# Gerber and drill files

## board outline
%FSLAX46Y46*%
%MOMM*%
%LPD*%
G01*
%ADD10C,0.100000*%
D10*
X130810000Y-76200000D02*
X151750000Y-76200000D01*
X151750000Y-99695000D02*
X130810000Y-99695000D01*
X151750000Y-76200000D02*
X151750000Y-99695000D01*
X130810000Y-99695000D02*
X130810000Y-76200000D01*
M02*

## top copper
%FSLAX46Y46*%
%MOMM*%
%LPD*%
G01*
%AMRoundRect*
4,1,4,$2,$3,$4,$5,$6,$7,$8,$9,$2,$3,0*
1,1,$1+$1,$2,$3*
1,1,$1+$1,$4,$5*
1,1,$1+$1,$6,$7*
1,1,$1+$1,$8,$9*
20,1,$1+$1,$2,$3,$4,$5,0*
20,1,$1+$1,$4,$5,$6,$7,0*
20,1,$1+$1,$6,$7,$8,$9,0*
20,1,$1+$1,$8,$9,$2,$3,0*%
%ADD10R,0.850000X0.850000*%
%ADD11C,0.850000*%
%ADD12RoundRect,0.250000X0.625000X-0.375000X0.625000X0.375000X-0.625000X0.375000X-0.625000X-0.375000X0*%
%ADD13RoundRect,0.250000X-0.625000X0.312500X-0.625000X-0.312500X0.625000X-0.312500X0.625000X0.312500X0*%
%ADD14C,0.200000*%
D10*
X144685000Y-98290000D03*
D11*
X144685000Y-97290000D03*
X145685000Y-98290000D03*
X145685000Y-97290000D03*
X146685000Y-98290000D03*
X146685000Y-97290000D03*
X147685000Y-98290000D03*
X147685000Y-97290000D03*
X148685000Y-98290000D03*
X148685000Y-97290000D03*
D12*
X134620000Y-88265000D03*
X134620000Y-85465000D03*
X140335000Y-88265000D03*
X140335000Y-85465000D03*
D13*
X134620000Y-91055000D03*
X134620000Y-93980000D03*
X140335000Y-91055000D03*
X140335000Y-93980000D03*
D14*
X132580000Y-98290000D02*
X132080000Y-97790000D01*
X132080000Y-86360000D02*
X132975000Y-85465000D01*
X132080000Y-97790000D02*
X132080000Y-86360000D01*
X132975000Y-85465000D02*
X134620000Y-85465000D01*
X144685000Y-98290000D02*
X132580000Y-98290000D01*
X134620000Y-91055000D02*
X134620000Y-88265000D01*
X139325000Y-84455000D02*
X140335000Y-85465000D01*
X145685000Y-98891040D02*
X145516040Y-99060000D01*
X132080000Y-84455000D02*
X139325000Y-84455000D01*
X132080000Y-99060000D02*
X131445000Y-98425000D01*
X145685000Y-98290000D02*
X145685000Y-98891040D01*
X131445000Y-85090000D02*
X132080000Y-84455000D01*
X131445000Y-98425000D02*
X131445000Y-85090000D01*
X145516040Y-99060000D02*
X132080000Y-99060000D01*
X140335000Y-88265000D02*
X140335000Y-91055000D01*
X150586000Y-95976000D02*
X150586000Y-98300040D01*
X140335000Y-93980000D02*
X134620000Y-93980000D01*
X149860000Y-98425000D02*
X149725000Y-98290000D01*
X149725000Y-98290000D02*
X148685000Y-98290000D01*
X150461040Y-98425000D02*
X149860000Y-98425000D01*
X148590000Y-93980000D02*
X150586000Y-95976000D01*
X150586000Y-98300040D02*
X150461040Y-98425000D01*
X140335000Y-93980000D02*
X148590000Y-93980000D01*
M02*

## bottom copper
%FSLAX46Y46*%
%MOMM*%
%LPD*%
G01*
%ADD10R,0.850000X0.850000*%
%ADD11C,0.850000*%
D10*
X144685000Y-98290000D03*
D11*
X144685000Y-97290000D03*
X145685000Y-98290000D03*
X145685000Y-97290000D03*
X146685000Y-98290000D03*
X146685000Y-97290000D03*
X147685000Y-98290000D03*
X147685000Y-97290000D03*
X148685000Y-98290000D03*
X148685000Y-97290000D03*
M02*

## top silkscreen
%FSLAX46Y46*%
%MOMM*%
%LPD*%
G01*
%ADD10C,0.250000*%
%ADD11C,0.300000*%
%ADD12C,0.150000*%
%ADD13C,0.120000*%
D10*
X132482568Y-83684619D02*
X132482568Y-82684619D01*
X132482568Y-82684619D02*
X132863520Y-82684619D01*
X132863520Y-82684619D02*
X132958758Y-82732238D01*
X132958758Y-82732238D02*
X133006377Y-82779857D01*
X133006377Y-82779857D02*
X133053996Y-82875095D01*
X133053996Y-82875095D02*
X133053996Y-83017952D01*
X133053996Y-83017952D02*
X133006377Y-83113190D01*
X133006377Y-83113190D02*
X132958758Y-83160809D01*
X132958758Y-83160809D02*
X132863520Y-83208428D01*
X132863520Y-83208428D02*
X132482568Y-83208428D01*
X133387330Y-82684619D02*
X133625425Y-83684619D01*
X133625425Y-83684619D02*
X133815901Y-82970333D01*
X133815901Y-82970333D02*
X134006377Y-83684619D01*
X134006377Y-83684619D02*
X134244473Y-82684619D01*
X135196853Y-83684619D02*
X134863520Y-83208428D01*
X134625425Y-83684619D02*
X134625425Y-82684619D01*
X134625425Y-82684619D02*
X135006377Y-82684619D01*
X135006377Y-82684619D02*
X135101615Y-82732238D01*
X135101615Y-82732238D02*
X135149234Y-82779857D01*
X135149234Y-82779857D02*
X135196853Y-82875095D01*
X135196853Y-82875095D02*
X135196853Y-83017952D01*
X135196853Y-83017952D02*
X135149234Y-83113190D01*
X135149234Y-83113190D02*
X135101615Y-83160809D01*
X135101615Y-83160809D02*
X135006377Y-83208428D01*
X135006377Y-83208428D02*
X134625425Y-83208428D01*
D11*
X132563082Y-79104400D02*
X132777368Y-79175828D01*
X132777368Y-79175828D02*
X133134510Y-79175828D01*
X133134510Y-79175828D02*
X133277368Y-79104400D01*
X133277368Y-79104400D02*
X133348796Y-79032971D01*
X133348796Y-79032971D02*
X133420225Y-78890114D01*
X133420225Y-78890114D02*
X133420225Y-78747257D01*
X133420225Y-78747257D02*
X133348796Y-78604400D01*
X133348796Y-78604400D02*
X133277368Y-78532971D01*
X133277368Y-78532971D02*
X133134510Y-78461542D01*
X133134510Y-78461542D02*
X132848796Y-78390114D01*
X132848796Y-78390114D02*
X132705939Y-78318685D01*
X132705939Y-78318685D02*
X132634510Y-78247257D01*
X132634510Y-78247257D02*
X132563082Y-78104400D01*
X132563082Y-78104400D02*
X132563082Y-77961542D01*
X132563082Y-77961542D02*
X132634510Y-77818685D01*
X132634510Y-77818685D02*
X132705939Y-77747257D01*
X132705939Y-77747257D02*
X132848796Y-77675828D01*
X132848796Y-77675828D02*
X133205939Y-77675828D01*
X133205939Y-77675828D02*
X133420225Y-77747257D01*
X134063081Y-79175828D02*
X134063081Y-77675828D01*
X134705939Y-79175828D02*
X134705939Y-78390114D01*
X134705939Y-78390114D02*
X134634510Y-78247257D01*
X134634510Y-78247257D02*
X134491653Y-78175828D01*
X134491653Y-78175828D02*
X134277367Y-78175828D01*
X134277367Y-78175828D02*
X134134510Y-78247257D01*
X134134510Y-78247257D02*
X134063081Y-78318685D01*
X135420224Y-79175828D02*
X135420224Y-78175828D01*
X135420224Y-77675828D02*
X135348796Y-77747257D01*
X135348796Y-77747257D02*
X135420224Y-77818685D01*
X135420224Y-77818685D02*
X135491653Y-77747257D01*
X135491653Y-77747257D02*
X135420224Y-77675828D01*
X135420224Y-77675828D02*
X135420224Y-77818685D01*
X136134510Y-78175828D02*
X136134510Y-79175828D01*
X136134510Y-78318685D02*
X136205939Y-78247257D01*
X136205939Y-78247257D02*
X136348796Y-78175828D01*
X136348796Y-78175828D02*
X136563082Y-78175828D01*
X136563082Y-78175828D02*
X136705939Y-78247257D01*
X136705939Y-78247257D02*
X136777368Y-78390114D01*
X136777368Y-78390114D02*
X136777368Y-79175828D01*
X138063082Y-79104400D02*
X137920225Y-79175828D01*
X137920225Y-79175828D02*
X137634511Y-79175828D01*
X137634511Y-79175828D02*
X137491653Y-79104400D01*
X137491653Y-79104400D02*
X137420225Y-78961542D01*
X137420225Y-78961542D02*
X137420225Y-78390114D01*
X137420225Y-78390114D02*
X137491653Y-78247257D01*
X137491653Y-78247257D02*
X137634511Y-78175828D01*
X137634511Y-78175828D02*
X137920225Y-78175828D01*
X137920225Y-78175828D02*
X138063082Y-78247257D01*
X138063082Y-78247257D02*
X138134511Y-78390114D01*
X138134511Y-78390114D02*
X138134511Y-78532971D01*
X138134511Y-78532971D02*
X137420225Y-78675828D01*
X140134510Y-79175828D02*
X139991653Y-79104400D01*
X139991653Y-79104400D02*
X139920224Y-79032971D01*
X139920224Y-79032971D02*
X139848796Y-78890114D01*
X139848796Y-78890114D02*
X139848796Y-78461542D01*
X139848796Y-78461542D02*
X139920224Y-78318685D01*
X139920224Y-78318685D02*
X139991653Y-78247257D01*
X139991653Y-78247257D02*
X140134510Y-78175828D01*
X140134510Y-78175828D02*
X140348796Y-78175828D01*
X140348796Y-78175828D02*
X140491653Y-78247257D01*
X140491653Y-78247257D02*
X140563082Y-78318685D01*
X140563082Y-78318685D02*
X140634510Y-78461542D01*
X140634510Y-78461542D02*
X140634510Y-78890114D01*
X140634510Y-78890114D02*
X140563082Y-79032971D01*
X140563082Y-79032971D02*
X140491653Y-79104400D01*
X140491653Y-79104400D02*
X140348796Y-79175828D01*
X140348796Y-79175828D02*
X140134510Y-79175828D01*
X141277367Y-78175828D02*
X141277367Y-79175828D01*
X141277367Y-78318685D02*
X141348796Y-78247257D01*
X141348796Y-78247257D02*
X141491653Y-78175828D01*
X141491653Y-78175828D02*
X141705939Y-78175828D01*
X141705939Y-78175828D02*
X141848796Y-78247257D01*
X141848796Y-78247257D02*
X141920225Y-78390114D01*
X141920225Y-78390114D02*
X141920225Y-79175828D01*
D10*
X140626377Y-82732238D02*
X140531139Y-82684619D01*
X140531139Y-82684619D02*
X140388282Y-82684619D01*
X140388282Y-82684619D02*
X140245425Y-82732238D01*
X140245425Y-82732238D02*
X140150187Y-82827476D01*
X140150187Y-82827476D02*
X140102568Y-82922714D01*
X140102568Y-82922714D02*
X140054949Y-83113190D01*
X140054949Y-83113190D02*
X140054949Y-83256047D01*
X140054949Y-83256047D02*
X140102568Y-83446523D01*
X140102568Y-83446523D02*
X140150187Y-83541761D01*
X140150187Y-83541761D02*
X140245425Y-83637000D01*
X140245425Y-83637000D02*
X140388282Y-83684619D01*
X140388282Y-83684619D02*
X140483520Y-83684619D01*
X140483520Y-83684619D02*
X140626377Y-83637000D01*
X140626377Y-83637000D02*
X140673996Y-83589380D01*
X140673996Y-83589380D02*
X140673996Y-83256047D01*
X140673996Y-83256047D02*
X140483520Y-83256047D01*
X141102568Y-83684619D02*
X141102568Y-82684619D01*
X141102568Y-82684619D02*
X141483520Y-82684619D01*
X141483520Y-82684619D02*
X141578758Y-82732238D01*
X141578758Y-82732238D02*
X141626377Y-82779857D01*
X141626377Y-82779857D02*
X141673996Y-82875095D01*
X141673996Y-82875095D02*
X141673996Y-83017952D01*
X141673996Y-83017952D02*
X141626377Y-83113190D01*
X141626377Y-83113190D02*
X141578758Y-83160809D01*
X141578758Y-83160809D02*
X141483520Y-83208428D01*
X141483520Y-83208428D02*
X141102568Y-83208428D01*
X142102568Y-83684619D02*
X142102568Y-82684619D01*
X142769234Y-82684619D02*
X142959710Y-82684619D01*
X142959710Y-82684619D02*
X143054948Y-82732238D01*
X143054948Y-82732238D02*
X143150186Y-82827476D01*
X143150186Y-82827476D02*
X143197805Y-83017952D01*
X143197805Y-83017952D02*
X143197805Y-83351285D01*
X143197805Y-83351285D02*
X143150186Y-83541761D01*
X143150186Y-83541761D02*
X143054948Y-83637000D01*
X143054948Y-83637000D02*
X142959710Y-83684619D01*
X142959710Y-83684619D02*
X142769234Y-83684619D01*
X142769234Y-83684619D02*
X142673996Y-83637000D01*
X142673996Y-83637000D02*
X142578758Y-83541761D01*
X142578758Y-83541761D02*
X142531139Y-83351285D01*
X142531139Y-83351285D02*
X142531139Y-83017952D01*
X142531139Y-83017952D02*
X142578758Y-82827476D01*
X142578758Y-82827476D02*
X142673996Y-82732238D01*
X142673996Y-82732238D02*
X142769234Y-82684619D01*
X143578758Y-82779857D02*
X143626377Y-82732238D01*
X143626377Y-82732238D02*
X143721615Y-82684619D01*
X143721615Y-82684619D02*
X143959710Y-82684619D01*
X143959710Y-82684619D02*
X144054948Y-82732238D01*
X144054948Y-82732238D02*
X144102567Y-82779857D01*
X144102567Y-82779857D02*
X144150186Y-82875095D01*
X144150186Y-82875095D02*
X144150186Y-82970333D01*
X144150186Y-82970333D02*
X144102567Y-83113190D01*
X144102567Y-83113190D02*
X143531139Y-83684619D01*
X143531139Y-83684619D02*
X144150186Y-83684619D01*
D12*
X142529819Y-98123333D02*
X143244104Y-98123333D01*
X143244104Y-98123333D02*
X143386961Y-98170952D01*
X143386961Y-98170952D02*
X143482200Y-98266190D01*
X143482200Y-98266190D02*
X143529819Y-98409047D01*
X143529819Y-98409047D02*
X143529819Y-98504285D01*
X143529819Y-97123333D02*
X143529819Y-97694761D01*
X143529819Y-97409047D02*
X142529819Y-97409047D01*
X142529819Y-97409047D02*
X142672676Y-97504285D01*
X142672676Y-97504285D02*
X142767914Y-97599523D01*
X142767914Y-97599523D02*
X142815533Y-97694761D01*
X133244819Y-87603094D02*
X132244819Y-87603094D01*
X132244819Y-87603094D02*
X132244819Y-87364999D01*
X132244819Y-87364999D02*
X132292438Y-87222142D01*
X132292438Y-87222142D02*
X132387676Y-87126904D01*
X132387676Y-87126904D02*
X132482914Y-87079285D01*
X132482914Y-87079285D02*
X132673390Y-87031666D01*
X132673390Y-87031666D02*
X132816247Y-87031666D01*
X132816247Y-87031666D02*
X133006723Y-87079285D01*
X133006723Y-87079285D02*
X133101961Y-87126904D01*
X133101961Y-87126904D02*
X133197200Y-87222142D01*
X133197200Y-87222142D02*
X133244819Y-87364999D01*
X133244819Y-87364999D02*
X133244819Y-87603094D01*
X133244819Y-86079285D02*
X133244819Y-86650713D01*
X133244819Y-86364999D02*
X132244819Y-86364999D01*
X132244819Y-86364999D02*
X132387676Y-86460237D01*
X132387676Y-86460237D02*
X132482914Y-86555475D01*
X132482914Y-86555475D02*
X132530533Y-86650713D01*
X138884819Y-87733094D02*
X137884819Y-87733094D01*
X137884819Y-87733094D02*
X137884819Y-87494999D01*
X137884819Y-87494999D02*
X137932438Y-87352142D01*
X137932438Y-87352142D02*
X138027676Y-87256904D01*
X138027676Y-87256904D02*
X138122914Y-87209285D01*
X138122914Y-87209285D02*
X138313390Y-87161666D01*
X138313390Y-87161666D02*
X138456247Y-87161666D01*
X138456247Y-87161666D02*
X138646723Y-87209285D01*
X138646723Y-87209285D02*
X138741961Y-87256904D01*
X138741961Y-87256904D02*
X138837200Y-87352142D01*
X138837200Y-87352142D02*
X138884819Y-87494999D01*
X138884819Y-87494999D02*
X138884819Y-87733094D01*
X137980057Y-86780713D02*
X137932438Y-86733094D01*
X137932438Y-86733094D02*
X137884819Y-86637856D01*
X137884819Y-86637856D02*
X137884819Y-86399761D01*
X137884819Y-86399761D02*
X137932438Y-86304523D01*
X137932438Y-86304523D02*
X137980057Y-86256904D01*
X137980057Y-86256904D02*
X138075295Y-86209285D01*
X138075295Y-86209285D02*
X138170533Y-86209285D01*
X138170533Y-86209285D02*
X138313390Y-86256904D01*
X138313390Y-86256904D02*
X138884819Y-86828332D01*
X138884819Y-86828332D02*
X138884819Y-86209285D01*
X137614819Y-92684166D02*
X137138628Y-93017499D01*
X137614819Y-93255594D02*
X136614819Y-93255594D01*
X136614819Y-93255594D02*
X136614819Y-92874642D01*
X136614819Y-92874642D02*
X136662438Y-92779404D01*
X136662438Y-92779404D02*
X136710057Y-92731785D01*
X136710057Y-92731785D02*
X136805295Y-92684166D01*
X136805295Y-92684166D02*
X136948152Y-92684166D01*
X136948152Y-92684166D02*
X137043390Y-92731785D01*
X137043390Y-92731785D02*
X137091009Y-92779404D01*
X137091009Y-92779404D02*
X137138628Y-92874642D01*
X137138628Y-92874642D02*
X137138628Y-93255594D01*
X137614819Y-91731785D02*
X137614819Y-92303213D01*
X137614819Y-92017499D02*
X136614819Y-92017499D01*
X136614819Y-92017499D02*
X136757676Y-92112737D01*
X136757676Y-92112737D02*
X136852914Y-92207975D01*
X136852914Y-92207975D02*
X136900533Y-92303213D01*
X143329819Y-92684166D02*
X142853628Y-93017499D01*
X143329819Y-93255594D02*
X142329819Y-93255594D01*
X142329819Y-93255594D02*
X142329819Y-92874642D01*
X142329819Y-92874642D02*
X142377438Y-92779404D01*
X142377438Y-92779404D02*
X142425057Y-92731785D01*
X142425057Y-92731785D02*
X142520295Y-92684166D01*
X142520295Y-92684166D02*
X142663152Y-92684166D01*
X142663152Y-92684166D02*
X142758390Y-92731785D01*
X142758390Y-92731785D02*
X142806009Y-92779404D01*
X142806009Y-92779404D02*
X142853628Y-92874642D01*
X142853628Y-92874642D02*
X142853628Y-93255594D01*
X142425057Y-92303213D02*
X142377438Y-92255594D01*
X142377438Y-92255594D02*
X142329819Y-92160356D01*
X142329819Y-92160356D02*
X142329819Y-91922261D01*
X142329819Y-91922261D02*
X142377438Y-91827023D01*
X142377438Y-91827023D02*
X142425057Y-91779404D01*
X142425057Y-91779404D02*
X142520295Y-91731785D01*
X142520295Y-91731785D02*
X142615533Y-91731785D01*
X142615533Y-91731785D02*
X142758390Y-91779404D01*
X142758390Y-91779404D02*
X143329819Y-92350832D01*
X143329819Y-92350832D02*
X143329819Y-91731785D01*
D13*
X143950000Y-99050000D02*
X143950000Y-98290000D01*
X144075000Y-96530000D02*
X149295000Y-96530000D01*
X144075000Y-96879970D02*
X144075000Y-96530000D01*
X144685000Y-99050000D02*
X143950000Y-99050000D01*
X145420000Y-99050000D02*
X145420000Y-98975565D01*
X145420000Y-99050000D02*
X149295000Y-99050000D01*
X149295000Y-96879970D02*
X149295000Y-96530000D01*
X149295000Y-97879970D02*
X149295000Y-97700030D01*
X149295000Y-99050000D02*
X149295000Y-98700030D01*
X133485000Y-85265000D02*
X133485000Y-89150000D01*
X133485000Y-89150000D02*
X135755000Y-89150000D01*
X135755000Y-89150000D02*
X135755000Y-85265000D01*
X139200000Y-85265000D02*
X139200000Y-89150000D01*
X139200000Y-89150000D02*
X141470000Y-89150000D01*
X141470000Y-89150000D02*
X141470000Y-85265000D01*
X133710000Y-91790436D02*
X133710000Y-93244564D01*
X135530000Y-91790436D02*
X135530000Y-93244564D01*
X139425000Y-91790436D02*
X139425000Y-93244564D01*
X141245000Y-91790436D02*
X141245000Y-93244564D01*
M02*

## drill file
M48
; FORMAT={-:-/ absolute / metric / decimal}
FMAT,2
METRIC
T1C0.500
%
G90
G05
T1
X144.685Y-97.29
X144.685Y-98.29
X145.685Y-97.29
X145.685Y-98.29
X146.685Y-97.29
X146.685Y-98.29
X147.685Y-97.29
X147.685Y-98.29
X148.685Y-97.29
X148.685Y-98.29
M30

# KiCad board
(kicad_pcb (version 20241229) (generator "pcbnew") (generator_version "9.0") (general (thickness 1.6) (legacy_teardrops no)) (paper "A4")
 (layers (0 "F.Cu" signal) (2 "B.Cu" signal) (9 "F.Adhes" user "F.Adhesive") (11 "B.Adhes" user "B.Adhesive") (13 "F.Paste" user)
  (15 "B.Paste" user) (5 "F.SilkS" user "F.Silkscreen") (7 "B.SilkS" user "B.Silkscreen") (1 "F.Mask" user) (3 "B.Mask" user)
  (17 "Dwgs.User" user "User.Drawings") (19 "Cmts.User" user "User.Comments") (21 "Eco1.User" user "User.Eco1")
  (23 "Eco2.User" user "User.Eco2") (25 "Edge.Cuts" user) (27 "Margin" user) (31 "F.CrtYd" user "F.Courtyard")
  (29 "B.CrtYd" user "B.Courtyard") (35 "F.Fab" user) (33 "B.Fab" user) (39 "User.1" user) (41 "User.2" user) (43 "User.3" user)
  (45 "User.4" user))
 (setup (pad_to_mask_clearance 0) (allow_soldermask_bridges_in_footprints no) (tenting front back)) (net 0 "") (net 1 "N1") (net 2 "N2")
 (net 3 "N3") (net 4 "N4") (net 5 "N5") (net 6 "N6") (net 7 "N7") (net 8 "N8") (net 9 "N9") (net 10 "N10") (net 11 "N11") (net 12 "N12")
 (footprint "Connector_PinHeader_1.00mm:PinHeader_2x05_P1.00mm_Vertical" (layer "F.Cu") (at 144.685 98.29 90)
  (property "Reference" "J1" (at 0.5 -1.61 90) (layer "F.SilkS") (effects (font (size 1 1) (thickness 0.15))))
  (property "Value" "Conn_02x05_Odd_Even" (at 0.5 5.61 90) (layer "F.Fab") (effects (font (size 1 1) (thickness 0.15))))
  (fp_line (start -0.76 -0.735) (end 0 -0.735) (stroke (width 0.12) (type solid)) (layer "F.SilkS"))
  (fp_line (start 1.76 -0.61) (end 1.76 4.61) (stroke (width 0.12) (type solid)) (layer "F.SilkS"))
  (fp_line (start 1.41003 -0.61) (end 1.76 -0.61) (stroke (width 0.12) (type solid)) (layer "F.SilkS"))
  (fp_line (start -0.76 0) (end -0.76 -0.735) (stroke (width 0.12) (type solid)) (layer "F.SilkS"))
  (fp_line (start -0.76 0.735) (end -0.685565 0.735) (stroke (width 0.12) (type solid)) (layer "F.SilkS"))
  (fp_line (start -0.76 0.735) (end -0.76 4.61) (stroke (width 0.12) (type solid)) (layer "F.SilkS"))
  (fp_line (start 1.41003 4.61) (end 1.76 4.61) (stroke (width 0.12) (type solid)) (layer "F.SilkS"))
  (fp_line (start 0.41003 4.61) (end 0.58997 4.61) (stroke (width 0.12) (type solid)) (layer "F.SilkS"))
  (fp_line (start -0.76 4.61) (end -0.41003 4.61) (stroke (width 0.12) (type solid)) (layer "F.SilkS"))
  (pad "1" thru_hole rect (at 0 0 90) (size 0.85 0.85) (drill 0.5) (layers "*.Cu" "*.Mask") (remove_unused_layers no) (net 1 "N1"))
  (pad "2" thru_hole circle (at 1 0 90) (size 0.85 0.85) (drill 0.5) (layers "*.Cu" "*.Mask") (remove_unused_layers no) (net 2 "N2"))
  (pad "3" thru_hole circle (at 0 1 90) (size 0.85 0.85) (drill 0.5) (layers "*.Cu" "*.Mask") (remove_unused_layers no) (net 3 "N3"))
  (pad "4" thru_hole circle (at 1 1 90) (size 0.85 0.85) (drill 0.5) (layers "*.Cu" "*.Mask") (remove_unused_layers no) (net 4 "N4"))
  (pad "5" thru_hole circle (at 0 2 90) (size 0.85 0.85) (drill 0.5) (layers "*.Cu" "*.Mask") (remove_unused_layers no) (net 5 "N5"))
  (pad "6" thru_hole circle (at 1 2 90) (size 0.85 0.85) (drill 0.5) (layers "*.Cu" "*.Mask") (remove_unused_layers no) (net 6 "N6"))
  (pad "7" thru_hole circle (at 0 3 90) (size 0.85 0.85) (drill 0.5) (layers "*.Cu" "*.Mask") (remove_unused_layers no) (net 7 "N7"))
  (pad "8" thru_hole circle (at 1 3 90) (size 0.85 0.85) (drill 0.5) (layers "*.Cu" "*.Mask") (remove_unused_layers no) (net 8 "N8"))
  (pad "9" thru_hole circle (at 0 4 90) (size 0.85 0.85) (drill 0.5) (layers "*.Cu" "*.Mask") (remove_unused_layers no) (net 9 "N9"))
  (pad "10" thru_hole circle (at 1 4 90) (size 0.85 0.85) (drill 0.5) (layers "*.Cu" "*.Mask") (remove_unused_layers no) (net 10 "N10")))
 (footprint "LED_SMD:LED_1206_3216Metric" (layer "F.Cu") (at 134.62 86.865 90)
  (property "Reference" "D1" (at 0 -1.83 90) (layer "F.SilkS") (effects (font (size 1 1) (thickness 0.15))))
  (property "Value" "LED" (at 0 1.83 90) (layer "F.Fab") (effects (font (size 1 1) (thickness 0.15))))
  (fp_line (start 1.6 -1.135) (end -2.285 -1.135) (stroke (width 0.12) (type solid)) (layer "F.SilkS"))
  (fp_line (start -2.285 -1.135) (end -2.285 1.135) (stroke (width 0.12) (type solid)) (layer "F.SilkS"))
  (fp_line (start -2.285 1.135) (end 1.6 1.135) (stroke (width 0.12) (type solid)) (layer "F.SilkS"))
  (pad "1" smd roundrect (at -1.4 0 90) (size 1.25 1.75) (layers "F.Cu" "F.Mask" "F.Paste") (roundrect_rratio 0.2) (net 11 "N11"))
  (pad "2" smd roundrect (at 1.4 0 90) (size 1.25 1.75) (layers "F.Cu" "F.Mask" "F.Paste") (roundrect_rratio 0.2) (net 1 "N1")))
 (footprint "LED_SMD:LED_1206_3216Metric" (layer "F.Cu") (at 140.335 86.865 90)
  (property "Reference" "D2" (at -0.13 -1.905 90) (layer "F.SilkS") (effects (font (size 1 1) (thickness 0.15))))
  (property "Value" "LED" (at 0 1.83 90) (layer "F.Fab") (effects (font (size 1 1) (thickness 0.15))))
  (fp_line (start 1.6 -1.135) (end -2.285 -1.135) (stroke (width 0.12) (type solid)) (layer "F.SilkS"))
  (fp_line (start -2.285 -1.135) (end -2.285 1.135) (stroke (width 0.12) (type solid)) (layer "F.SilkS"))
  (fp_line (start -2.285 1.135) (end 1.6 1.135) (stroke (width 0.12) (type solid)) (layer "F.SilkS"))
  (pad "1" smd roundrect (at -1.4 0 90) (size 1.25 1.75) (layers "F.Cu" "F.Mask" "F.Paste") (roundrect_rratio 0.2) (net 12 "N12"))
  (pad "2" smd roundrect (at 1.4 0 90) (size 1.25 1.75) (layers "F.Cu" "F.Mask" "F.Paste") (roundrect_rratio 0.2) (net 3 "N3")))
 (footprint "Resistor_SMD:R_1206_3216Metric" (layer "F.Cu") (at 134.62 92.5175 -90)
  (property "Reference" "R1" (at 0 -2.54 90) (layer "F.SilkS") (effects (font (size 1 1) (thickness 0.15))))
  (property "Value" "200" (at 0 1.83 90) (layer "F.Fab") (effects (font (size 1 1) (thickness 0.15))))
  (fp_line (start -0.727064 0.91) (end 0.727064 0.91) (stroke (width 0.12) (type solid)) (layer "F.SilkS"))
  (fp_line (start -0.727064 -0.91) (end 0.727064 -0.91) (stroke (width 0.12) (type solid)) (layer "F.SilkS"))
  (pad "1" smd roundrect (at -1.4625 0 270) (size 1.125 1.75) (layers "F.Cu" "F.Mask" "F.Paste") (roundrect_rratio 0.222222) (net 11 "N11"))
  (pad "2" smd roundrect (at 1.4625 0 270) (size 1.125 1.75) (layers "F.Cu" "F.Mask" "F.Paste") (roundrect_rratio 0.222222) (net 9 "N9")))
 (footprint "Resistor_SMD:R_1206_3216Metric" (layer "F.Cu") (at 140.335 92.5175 -90)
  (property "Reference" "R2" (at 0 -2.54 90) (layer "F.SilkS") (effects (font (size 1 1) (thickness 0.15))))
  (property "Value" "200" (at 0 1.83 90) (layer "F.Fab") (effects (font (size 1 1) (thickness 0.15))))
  (fp_line (start -0.727064 0.91) (end 0.727064 0.91) (stroke (width 0.12) (type solid)) (layer "F.SilkS"))
  (fp_line (start -0.727064 -0.91) (end 0.727064 -0.91) (stroke (width 0.12) (type solid)) (layer "F.SilkS"))
  (pad "1" smd roundrect (at -1.4625 0 270) (size 1.125 1.75) (layers "F.Cu" "F.Mask" "F.Paste") (roundrect_rratio 0.222222) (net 12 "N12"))
  (pad "2" smd roundrect (at 1.4625 0 270) (size 1.125 1.75) (layers "F.Cu" "F.Mask" "F.Paste") (roundrect_rratio 0.222222) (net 9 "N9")))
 (gr_line (start 130.81 76.2) (end 151.75 76.2) (stroke (width 0.1) (type solid)) (layer "Edge.Cuts"))
 (gr_line (start 151.75 99.695) (end 130.81 99.695) (stroke (width 0.1) (type solid)) (layer "Edge.Cuts"))
 (gr_line (start 151.75 76.2) (end 151.75 99.695) (stroke (width 0.1) (type solid)) (layer "Edge.Cuts"))
 (gr_line (start 130.81 99.695) (end 130.81 76.2) (stroke (width 0.1) (type solid)) (layer "Edge.Cuts"))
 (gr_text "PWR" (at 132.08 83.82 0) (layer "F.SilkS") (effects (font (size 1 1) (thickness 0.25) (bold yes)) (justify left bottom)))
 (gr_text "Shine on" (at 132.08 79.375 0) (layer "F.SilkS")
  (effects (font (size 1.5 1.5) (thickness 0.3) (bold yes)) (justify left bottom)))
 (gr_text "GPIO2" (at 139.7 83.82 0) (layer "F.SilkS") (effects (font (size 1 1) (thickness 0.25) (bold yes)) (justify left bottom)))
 (segment (start 132.58 98.29) (end 132.08 97.79) (width 0.2) (layer "F.Cu") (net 1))
 (segment (start 132.08 86.36) (end 132.975 85.465) (width 0.2) (layer "F.Cu") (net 1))
 (segment (start 132.08 97.79) (end 132.08 86.36) (width 0.2) (layer "F.Cu") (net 1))
 (segment (start 132.975 85.465) (end 134.62 85.465) (width 0.2) (layer "F.Cu") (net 1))
 (segment (start 144.685 98.29) (end 132.58 98.29) (width 0.2) (layer "F.Cu") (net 1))
 (segment (start 134.62 91.055) (end 134.62 88.265) (width 0.2) (layer "F.Cu") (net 11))
 (segment (start 139.325 84.455) (end 140.335 85.465) (width 0.2) (layer "F.Cu") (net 3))
 (segment (start 145.685 98.89104) (end 145.51604 99.06) (width 0.2) (layer "F.Cu") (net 3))
 (segment (start 132.08 84.455) (end 139.325 84.455) (width 0.2) (layer "F.Cu") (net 3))
 (segment (start 132.08 99.06) (end 131.445 98.425) (width 0.2) (layer "F.Cu") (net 3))
 (segment (start 145.685 98.29) (end 145.685 98.89104) (width 0.2) (layer "F.Cu") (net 3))
 (segment (start 131.445 85.09) (end 132.08 84.455) (width 0.2) (layer "F.Cu") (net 3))
 (segment (start 131.445 98.425) (end 131.445 85.09) (width 0.2) (layer "F.Cu") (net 3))
 (segment (start 145.51604 99.06) (end 132.08 99.06) (width 0.2) (layer "F.Cu") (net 3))
 (segment (start 140.335 88.265) (end 140.335 91.055) (width 0.2) (layer "F.Cu") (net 12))
 (segment (start 150.586 95.976) (end 150.586 98.30004) (width 0.2) (layer "F.Cu") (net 9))
 (segment (start 140.335 93.98) (end 134.62 93.98) (width 0.2) (layer "F.Cu") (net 9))
 (segment (start 149.86 98.425) (end 149.725 98.29) (width 0.2) (layer "F.Cu") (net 9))
 (segment (start 149.725 98.29) (end 148.685 98.29) (width 0.2) (layer "F.Cu") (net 9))
 (segment (start 150.46104 98.425) (end 149.86 98.425) (width 0.2) (layer "F.Cu") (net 9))
 (segment (start 148.59 93.98) (end 150.586 95.976) (width 0.2) (layer "F.Cu") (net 9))
 (segment (start 150.586 98.30004) (end 150.46104 98.425) (width 0.2) (layer "F.Cu") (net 9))
 (segment (start 140.335 93.98) (end 148.59 93.98) (width 0.2) (layer "F.Cu") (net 9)))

